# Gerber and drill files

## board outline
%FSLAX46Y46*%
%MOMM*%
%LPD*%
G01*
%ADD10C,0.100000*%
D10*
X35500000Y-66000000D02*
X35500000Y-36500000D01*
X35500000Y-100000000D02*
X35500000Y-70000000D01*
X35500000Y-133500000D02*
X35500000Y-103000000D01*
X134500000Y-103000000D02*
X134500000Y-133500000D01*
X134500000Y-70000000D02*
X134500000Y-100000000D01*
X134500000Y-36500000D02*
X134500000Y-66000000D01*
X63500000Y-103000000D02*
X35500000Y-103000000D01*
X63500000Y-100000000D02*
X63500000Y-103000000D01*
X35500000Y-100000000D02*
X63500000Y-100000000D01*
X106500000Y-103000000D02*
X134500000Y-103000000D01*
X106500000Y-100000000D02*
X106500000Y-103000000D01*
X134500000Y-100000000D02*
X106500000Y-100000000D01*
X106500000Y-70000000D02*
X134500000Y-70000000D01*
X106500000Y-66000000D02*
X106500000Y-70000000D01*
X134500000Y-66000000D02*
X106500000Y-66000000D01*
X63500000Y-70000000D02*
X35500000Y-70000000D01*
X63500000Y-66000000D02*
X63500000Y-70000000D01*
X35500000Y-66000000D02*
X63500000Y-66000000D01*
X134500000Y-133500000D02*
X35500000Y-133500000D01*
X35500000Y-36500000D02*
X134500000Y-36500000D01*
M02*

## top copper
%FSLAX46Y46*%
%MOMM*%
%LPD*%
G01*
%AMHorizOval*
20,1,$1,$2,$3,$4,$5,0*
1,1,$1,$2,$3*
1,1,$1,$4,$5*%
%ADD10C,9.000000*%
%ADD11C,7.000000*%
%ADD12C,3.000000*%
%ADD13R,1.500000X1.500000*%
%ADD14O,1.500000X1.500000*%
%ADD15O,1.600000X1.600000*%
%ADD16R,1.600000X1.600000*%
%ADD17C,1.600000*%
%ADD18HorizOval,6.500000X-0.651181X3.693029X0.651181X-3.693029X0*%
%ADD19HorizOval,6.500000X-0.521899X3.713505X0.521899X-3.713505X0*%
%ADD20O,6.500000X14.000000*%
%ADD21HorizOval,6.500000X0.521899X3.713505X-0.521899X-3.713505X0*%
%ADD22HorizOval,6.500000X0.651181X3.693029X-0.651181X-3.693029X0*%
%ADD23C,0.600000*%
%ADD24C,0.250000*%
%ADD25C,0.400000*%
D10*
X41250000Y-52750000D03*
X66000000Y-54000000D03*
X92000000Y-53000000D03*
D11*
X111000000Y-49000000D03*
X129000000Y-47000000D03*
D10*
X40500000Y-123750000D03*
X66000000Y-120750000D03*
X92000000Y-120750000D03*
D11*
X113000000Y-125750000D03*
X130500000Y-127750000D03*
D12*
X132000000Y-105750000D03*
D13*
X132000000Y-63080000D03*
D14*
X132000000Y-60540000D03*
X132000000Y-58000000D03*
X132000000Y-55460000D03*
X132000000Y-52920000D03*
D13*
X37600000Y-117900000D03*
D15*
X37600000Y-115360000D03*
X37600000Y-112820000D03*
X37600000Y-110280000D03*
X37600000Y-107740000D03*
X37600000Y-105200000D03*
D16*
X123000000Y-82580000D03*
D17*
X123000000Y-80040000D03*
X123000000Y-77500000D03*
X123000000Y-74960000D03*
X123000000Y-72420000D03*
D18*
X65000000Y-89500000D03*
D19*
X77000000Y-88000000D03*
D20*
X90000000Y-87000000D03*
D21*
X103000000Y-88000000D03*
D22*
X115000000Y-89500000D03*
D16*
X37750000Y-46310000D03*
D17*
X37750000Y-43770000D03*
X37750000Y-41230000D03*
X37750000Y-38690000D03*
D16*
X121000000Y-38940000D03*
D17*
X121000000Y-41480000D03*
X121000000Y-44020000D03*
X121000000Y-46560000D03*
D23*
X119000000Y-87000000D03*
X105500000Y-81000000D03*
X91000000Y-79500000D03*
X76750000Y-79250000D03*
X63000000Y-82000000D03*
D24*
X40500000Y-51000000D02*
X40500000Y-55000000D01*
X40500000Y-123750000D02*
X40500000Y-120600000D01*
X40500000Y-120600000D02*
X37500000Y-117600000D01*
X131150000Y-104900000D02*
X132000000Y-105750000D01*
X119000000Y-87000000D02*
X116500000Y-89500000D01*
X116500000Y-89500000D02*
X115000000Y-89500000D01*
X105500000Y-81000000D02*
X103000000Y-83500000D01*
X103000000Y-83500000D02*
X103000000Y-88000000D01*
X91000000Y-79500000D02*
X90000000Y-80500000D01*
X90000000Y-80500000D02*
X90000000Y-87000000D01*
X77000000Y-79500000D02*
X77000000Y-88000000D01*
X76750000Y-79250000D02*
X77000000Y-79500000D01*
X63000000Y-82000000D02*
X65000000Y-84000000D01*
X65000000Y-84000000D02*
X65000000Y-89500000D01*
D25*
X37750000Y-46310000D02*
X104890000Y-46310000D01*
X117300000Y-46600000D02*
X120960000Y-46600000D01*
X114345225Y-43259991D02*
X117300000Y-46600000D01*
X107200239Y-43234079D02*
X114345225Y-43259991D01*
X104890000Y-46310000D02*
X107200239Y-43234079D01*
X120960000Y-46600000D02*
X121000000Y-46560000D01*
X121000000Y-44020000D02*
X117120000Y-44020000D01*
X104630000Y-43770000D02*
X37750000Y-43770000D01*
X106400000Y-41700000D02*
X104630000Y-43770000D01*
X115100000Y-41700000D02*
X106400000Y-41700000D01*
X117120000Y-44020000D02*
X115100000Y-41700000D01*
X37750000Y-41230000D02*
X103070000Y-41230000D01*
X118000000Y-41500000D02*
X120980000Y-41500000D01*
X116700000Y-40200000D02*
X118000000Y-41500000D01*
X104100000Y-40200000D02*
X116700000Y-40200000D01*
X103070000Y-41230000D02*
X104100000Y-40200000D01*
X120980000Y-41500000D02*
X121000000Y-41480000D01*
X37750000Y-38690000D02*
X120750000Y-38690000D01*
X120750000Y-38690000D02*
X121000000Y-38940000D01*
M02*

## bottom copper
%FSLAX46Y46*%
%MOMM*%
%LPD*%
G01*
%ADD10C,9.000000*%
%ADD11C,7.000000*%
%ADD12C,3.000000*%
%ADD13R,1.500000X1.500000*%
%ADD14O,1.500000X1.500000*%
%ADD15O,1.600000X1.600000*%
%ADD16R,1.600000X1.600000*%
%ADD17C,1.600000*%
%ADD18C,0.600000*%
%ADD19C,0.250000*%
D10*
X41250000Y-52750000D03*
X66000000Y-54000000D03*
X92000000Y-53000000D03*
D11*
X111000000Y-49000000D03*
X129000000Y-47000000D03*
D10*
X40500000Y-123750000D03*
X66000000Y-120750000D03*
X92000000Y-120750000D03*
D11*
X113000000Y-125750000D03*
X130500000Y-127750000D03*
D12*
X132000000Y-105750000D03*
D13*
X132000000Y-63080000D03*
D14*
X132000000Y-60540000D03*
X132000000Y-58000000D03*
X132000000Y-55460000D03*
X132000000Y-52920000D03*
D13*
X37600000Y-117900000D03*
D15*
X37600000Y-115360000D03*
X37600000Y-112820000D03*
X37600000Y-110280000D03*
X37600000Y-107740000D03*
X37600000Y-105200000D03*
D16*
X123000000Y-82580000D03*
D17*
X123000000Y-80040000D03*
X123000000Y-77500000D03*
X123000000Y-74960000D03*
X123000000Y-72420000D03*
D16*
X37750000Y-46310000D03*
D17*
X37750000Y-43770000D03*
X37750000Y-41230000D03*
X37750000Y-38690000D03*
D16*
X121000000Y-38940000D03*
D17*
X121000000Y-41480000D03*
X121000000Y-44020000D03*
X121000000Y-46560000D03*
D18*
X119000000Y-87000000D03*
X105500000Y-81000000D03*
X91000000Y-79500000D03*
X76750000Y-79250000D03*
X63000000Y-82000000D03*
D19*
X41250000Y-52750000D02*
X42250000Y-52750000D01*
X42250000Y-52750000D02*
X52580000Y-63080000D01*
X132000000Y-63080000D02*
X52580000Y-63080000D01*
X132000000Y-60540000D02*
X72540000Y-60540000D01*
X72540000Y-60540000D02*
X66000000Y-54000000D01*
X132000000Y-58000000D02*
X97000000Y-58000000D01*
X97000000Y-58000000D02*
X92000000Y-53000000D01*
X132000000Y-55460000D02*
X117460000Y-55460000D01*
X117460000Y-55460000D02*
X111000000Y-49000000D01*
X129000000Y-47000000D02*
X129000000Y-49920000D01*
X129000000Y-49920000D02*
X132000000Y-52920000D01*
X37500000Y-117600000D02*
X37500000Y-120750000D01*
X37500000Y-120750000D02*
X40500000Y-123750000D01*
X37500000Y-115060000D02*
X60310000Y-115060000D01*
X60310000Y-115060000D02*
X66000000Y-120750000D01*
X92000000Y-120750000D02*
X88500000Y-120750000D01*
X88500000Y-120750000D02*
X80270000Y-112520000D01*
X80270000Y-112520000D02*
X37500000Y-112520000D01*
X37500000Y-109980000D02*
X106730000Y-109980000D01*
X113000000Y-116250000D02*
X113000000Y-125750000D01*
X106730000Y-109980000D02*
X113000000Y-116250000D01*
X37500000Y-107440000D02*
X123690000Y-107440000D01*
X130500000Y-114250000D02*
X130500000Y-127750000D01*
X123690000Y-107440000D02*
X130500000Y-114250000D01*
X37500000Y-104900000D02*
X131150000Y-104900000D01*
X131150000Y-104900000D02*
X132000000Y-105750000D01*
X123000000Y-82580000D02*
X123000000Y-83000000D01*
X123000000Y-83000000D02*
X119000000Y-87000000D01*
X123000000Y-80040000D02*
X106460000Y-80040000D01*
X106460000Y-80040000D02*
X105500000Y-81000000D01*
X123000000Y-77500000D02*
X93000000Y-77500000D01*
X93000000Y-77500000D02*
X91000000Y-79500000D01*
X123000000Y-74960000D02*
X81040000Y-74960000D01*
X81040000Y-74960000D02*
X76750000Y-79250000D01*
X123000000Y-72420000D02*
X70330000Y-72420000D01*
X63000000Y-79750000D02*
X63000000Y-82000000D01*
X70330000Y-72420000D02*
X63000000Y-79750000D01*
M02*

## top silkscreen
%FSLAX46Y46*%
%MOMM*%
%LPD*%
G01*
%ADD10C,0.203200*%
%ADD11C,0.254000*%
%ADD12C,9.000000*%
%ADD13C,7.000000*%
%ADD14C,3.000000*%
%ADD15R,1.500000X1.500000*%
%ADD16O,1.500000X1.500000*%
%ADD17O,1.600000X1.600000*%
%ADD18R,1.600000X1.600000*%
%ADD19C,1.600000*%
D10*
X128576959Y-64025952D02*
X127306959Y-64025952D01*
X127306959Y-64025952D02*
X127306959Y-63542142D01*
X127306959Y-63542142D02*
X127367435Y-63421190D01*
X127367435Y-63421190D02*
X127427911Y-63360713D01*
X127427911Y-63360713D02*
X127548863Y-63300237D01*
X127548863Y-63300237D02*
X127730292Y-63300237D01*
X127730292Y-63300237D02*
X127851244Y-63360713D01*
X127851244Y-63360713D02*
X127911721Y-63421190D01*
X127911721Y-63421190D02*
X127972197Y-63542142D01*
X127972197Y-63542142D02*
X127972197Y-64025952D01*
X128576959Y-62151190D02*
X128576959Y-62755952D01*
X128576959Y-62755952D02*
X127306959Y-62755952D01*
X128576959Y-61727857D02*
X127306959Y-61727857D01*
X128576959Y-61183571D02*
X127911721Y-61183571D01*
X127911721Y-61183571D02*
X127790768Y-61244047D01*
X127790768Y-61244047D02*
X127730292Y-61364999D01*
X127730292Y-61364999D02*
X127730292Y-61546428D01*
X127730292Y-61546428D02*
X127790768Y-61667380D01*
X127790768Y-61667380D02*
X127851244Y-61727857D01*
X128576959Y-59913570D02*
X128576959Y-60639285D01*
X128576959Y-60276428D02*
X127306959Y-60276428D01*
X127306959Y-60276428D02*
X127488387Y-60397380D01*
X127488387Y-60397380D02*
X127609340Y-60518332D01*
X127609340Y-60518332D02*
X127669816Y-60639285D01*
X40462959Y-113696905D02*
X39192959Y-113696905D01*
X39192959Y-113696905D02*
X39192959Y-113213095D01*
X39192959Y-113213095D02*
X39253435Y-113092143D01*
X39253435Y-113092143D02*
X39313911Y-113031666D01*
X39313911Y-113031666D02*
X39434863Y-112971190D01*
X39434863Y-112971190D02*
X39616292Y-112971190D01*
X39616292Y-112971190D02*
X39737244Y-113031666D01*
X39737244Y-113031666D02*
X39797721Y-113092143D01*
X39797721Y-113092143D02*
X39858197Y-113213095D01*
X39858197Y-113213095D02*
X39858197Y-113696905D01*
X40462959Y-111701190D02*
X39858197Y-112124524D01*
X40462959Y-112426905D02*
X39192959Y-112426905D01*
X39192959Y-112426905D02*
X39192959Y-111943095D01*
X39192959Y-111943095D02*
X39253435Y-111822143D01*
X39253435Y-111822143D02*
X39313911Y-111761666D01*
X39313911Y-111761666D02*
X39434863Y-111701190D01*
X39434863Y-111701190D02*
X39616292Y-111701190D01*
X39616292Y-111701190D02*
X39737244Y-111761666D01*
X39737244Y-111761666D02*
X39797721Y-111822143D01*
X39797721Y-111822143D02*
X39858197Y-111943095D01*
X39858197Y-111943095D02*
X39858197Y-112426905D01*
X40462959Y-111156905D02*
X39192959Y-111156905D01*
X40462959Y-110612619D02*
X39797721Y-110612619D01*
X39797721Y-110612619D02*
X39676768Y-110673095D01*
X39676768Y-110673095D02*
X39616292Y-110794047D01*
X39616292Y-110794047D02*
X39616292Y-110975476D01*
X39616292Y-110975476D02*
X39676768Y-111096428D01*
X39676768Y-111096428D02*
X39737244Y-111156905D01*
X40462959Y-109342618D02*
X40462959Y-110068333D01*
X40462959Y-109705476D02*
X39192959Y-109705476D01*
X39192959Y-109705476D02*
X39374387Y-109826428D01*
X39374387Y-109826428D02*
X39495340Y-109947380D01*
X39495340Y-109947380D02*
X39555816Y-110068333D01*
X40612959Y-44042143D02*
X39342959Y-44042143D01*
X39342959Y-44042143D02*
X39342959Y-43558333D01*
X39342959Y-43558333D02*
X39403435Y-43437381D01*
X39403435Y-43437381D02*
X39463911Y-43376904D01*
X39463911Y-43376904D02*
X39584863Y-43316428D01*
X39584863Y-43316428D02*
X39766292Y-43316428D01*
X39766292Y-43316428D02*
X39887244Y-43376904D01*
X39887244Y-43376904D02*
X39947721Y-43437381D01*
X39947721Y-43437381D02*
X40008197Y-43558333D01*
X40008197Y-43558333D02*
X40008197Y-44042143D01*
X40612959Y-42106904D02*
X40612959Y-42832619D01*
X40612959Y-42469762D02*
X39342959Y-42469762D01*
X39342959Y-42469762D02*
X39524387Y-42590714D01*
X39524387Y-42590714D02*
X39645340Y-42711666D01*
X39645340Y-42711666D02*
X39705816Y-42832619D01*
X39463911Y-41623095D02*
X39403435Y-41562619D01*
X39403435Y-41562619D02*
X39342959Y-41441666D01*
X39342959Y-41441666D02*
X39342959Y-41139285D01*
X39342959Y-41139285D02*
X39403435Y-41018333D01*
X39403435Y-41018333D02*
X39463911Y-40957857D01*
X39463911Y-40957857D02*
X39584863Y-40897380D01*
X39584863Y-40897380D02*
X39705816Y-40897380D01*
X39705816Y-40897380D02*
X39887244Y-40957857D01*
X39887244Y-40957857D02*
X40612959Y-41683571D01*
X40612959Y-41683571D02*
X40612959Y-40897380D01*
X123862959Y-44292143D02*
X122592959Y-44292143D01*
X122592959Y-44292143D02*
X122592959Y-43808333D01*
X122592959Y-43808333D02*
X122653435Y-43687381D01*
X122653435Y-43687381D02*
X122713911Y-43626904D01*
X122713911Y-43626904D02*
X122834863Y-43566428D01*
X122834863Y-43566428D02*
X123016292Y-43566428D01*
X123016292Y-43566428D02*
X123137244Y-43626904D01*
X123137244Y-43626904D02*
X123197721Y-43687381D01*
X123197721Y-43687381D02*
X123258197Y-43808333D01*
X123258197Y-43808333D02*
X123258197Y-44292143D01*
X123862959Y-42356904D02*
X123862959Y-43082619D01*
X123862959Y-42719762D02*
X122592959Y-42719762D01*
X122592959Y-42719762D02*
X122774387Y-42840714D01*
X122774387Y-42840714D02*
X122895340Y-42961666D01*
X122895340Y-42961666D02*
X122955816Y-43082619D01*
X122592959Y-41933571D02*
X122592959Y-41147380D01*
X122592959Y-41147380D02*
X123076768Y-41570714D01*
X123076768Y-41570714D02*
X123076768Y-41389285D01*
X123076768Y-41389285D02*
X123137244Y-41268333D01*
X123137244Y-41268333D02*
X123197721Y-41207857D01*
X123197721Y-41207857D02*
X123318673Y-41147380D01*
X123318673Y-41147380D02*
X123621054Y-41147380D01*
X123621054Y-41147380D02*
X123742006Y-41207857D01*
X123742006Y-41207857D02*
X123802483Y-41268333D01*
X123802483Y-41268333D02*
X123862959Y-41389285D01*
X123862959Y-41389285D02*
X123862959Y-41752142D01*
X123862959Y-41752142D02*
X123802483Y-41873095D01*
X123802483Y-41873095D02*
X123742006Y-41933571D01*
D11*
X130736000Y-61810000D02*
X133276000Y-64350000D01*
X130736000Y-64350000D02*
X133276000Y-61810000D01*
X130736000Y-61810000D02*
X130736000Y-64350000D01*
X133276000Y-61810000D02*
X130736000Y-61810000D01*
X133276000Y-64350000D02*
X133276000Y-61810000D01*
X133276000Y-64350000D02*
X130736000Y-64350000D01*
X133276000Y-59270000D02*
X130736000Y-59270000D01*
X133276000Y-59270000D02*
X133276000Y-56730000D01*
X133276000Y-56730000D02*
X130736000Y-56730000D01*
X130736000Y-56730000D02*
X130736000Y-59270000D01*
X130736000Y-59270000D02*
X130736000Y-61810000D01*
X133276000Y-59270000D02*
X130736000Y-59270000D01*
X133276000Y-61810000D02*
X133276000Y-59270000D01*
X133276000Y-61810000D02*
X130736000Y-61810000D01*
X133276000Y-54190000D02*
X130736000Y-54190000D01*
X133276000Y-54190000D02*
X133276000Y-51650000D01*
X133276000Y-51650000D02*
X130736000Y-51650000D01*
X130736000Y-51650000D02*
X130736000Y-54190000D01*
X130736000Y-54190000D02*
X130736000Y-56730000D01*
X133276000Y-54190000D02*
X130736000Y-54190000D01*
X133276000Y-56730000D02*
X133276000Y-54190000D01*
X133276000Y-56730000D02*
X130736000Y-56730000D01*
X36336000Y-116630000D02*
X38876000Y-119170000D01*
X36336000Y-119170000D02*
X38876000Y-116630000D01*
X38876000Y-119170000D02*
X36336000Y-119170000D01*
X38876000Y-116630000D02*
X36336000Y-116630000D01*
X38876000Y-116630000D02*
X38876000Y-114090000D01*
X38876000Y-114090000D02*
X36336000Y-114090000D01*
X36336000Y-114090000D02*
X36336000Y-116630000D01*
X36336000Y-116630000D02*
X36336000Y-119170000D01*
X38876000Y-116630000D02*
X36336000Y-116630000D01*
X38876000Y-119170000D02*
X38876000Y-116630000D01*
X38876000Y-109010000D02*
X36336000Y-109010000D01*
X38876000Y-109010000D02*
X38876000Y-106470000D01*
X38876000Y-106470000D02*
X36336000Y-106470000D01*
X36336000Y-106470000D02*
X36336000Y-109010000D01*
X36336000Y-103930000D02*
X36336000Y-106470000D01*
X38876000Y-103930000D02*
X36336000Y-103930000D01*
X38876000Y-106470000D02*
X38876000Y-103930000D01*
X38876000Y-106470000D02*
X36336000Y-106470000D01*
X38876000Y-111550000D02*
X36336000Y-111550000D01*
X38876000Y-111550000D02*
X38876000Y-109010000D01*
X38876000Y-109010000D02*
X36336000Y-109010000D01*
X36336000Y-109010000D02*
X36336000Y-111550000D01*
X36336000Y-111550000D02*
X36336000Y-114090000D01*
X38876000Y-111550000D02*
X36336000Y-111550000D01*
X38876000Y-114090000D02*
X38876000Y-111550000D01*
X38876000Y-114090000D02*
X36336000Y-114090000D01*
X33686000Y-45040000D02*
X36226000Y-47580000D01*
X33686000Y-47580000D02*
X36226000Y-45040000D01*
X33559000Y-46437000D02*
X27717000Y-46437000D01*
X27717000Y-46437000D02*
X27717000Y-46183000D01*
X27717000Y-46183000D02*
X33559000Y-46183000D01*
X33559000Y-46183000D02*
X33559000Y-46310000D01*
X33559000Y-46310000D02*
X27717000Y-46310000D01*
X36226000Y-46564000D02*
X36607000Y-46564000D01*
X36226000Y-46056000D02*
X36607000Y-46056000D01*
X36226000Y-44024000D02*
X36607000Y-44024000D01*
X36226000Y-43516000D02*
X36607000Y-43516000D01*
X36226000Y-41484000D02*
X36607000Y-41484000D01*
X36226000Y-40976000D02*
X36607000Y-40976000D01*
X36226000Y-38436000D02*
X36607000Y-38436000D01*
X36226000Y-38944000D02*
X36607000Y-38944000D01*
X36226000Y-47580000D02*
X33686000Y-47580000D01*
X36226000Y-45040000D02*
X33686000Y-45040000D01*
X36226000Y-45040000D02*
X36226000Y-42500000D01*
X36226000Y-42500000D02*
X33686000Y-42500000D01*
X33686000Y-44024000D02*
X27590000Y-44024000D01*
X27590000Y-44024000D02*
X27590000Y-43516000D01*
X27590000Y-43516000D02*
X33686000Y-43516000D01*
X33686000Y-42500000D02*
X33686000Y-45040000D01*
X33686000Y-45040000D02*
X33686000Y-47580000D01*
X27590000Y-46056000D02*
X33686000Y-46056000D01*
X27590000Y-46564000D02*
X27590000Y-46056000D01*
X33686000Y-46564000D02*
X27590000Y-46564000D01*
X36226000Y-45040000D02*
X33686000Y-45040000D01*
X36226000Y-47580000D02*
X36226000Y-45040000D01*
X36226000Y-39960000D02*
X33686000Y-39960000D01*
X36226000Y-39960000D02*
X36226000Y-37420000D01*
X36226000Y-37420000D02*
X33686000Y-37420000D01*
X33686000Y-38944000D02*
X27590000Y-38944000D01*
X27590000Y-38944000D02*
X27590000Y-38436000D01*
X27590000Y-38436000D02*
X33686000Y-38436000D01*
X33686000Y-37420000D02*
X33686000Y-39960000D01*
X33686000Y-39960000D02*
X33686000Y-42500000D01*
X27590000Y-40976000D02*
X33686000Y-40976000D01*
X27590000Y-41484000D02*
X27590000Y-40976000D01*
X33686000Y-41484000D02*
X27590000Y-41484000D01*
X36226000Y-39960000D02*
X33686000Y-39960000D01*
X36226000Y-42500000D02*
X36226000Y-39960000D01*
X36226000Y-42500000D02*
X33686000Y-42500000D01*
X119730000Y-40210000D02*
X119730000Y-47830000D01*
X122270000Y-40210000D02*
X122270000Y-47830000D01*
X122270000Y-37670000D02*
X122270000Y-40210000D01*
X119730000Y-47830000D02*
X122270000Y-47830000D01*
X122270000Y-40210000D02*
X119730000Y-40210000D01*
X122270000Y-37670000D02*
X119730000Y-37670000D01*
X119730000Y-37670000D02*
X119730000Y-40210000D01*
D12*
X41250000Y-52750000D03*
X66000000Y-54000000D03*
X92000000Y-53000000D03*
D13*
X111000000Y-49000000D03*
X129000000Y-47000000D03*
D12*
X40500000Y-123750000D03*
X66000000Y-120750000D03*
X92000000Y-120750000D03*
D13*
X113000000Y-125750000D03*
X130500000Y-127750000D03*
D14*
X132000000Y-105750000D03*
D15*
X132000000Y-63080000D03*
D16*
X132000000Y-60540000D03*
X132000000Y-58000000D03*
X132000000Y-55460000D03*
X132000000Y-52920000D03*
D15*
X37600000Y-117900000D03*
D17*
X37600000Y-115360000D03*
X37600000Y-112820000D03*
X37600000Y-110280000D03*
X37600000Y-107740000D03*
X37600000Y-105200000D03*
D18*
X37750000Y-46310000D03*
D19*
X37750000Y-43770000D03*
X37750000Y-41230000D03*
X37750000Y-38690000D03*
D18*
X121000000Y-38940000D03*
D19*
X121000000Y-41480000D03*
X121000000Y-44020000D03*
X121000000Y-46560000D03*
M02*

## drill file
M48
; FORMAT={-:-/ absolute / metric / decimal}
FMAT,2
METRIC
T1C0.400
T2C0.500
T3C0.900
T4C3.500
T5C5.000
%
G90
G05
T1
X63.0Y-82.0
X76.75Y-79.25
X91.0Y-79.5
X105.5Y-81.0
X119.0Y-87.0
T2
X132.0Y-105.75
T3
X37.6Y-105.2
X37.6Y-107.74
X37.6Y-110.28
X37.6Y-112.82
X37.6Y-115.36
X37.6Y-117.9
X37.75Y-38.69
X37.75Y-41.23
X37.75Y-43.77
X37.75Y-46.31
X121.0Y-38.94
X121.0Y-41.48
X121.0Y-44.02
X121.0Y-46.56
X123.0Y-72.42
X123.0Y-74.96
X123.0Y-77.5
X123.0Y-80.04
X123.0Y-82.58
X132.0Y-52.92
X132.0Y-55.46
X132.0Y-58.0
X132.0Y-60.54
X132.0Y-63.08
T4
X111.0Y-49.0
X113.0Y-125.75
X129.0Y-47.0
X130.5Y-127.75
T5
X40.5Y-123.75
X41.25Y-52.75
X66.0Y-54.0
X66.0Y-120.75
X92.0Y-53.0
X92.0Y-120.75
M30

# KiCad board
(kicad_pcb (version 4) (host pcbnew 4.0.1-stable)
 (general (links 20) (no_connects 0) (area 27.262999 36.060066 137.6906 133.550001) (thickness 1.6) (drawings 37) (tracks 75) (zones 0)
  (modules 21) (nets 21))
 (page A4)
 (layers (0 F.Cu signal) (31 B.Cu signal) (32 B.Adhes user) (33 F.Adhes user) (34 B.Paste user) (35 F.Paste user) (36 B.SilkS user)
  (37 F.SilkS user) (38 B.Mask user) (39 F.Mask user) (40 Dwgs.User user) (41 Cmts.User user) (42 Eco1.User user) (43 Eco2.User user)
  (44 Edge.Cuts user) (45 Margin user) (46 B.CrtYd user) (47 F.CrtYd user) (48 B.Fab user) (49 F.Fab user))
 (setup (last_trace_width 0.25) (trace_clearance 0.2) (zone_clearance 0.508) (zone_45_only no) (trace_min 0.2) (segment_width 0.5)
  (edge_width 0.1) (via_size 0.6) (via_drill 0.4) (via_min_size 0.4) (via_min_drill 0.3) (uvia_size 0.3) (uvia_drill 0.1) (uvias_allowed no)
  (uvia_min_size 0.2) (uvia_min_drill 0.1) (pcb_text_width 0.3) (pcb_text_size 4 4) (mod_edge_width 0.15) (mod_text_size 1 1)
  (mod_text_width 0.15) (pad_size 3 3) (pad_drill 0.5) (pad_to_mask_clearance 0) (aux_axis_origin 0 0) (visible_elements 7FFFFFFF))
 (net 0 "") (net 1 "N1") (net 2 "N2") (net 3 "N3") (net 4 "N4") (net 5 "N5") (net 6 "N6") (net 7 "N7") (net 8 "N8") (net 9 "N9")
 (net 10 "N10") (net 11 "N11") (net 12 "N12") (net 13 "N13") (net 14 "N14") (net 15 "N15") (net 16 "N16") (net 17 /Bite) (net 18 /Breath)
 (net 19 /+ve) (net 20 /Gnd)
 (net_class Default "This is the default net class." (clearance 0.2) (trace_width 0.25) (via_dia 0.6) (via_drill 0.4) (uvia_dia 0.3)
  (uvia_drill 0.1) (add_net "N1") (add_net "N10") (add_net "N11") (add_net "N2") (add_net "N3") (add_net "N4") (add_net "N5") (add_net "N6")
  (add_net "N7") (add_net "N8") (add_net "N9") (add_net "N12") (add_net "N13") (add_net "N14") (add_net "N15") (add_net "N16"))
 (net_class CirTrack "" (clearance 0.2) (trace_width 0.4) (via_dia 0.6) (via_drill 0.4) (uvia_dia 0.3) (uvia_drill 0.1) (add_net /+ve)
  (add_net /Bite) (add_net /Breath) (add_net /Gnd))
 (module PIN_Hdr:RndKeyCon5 (layer F.Cu) (at 41.25 52.75)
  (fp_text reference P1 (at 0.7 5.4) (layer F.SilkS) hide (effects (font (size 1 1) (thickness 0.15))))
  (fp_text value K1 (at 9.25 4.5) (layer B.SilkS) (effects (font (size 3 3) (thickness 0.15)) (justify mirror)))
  (pad 1 thru_hole circle (at 0 0) (size 9 9) (drill 5) (layers *.Cu *.Mask F.SilkS) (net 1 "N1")))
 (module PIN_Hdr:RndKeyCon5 (layer F.Cu) (at 66 54)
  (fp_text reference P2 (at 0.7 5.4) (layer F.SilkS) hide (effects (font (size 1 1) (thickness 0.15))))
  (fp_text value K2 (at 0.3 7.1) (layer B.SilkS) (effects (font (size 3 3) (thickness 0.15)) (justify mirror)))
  (pad 1 thru_hole circle (at 0 0) (size 9 9) (drill 5) (layers *.Cu *.Mask F.SilkS) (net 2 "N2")))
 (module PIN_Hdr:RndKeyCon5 (layer F.Cu) (at 92 53)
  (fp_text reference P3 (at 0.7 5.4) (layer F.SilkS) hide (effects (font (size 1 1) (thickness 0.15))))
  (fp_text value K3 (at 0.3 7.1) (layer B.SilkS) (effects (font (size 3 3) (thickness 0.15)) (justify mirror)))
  (pad 1 thru_hole circle (at 0 0) (size 9 9) (drill 5) (layers *.Cu *.Mask F.SilkS) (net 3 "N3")))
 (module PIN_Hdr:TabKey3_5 (layer F.Cu) (at 111 49)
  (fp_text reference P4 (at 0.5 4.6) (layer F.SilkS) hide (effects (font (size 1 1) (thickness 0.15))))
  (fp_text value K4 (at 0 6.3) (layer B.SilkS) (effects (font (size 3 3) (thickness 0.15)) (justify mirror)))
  (pad 1 thru_hole circle (at 0 0) (size 7 7) (drill 3.5) (layers *.Cu *.Mask F.SilkS) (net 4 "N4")))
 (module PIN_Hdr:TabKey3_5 (layer F.Cu) (at 129 47)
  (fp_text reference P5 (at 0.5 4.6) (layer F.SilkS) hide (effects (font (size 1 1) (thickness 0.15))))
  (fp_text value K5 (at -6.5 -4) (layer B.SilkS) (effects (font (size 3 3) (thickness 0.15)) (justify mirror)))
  (pad 1 thru_hole circle (at 0 0) (size 7 7) (drill 3.5) (layers *.Cu *.Mask F.SilkS) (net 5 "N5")))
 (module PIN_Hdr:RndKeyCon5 (layer F.Cu) (at 40.5 123.75)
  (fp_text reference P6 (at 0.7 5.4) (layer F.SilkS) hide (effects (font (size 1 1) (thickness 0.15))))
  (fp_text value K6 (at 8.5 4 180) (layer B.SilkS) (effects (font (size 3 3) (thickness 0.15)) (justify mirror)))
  (pad 1 thru_hole circle (at 0 0) (size 9 9) (drill 5) (layers *.Cu *.Mask F.SilkS) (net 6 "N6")))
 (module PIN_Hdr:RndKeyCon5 (layer F.Cu) (at 66 120.75)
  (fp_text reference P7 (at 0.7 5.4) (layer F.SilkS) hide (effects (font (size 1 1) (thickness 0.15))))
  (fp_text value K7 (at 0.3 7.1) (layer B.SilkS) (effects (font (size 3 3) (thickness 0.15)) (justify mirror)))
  (pad 1 thru_hole circle (at 0 0) (size 9 9) (drill 5) (layers *.Cu *.Mask F.SilkS) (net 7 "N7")))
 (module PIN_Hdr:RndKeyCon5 (layer F.Cu) (at 92 120.75)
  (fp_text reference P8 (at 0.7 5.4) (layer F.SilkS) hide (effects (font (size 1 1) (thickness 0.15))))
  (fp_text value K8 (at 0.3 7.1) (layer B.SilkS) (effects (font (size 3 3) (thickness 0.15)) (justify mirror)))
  (pad 1 thru_hole circle (at 0 0) (size 9 9) (drill 5) (layers *.Cu *.Mask F.SilkS) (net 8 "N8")))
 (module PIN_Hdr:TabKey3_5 (layer F.Cu) (at 113 125.75)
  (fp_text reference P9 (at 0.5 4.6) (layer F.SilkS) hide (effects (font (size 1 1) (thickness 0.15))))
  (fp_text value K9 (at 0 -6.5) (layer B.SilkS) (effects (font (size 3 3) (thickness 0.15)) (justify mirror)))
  (pad 1 thru_hole circle (at 0 0) (size 7 7) (drill 3.5) (layers *.Cu *.Mask F.SilkS) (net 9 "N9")))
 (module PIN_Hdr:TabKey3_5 (layer F.Cu) (at 130.5 127.75)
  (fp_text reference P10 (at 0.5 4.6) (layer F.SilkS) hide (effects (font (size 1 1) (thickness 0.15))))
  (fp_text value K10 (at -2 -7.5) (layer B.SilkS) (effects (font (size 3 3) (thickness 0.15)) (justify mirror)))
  (pad 1 thru_hole circle (at 0 0) (size 7 7) (drill 3.5) (layers *.Cu *.Mask F.SilkS) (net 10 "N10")))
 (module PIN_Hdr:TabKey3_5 (layer F.Cu) (at 132 105.75)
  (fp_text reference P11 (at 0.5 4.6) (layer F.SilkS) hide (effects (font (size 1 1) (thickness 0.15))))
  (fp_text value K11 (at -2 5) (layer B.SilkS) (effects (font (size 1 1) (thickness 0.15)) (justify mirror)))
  (pad 1 thru_hole circle (at 0 0) (size 3 3) (drill 0.5) (layers *.Cu *.Mask F.SilkS) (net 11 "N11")))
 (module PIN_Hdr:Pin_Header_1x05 (layer F.Cu) (at 132 58 90)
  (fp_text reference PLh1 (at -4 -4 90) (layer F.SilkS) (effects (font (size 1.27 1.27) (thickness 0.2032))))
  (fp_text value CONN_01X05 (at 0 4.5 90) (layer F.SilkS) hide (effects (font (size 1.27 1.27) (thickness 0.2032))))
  (fp_line (start -3.81 -1.264) (end -6.35 1.276) (layer F.SilkS) (width 0.254))
  (fp_line (start -6.35 -1.264) (end -3.81 1.276) (layer F.SilkS) (width 0.254))
  (fp_line (start -3.81 -1.264) (end -6.35 -1.264) (layer F.SilkS) (width 0.254))
  (fp_line (start -3.81 1.276) (end -3.81 -1.264) (layer F.SilkS) (width 0.254))
  (fp_line (start -6.35 1.276) (end -3.81 1.276) (layer F.SilkS) (width 0.254))
  (fp_line (start -6.35 1.276) (end -6.35 -1.264) (layer F.SilkS) (width 0.254))
  (fp_line (start -1.27 1.276) (end -1.27 -1.264) (layer F.SilkS) (width 0.254))
  (fp_line (start -1.27 1.276) (end 1.27 1.276) (layer F.SilkS) (width 0.254))
  (fp_line (start 1.27 1.276) (end 1.27 -1.264) (layer F.SilkS) (width 0.254))
  (fp_line (start 1.27 -1.264) (end -1.27 -1.264) (layer F.SilkS) (width 0.254))
  (fp_line (start -1.27 -1.264) (end -3.81 -1.264) (layer F.SilkS) (width 0.254))
  (fp_line (start -1.27 1.276) (end -1.27 -1.264) (layer F.SilkS) (width 0.254))
  (fp_line (start -3.81 1.276) (end -1.27 1.276) (layer F.SilkS) (width 0.254))
  (fp_line (start -3.81 1.276) (end -3.81 -1.264) (layer F.SilkS) (width 0.254))
  (fp_line (start 3.81 1.276) (end 3.81 -1.264) (layer F.SilkS) (width 0.254))
  (fp_line (start 3.81 1.276) (end 6.35 1.276) (layer F.SilkS) (width 0.254))
  (fp_line (start 6.35 1.276) (end 6.35 -1.264) (layer F.SilkS) (width 0.254))
  (fp_line (start 6.35 -1.264) (end 3.81 -1.264) (layer F.SilkS) (width 0.254))
  (fp_line (start 3.81 -1.264) (end 1.27 -1.264) (layer F.SilkS) (width 0.254))
  (fp_line (start 3.81 1.276) (end 3.81 -1.264) (layer F.SilkS) (width 0.254))
  (fp_line (start 1.27 1.276) (end 3.81 1.276) (layer F.SilkS) (width 0.254))
  (fp_line (start 1.27 1.276) (end 1.27 -1.264) (layer F.SilkS) (width 0.254))
  (pad 1 thru_hole rect (at -5.08 0 90) (size 1.5 1.5) (drill 0.9) (layers *.Cu *.Mask F.SilkS) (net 1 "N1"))
  (pad 2 thru_hole oval (at -2.54 0 90) (size 1.5 1.5) (drill 0.9) (layers *.Cu *.Mask F.SilkS) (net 2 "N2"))
  (pad 3 thru_hole oval (at 0 0 90) (size 1.5 1.5) (drill 0.9) (layers *.Cu *.Mask F.SilkS) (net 3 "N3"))
  (pad 4 thru_hole oval (at 2.54 0 90) (size 1.5 1.5) (drill 0.9) (layers *.Cu *.Mask F.SilkS) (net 4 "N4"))
  (pad 5 thru_hole oval (at 5.08 0 90) (size 1.5 1.5) (drill 0.9) (layers *.Cu *.Mask F.SilkS) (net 5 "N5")))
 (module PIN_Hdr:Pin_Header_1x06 (layer F.Cu) (at 37.6 111.55 90)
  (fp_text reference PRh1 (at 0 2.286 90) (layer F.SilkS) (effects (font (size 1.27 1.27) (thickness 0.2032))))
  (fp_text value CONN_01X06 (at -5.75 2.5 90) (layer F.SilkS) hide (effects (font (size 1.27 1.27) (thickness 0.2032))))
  (fp_line (start -5.08 -1.264) (end -7.62 1.276) (layer F.SilkS) (width 0.254))
  (fp_line (start -7.62 -1.264) (end -5.08 1.276) (layer F.SilkS) (width 0.254))
  (fp_line (start -7.62 1.276) (end -7.62 -1.264) (layer F.SilkS) (width 0.254))
  (fp_line (start -5.08 1.276) (end -5.08 -1.264) (layer F.SilkS) (width 0.254))
  (fp_line (start -5.08 1.276) (end -2.54 1.276) (layer F.SilkS) (width 0.254))
  (fp_line (start -2.54 1.276) (end -2.54 -1.264) (layer F.SilkS) (width 0.254))
  (fp_line (start -2.54 -1.264) (end -5.08 -1.264) (layer F.SilkS) (width 0.254))
  (fp_line (start -5.08 -1.264) (end -7.62 -1.264) (layer F.SilkS) (width 0.254))
  (fp_line (start -5.08 1.276) (end -5.08 -1.264) (layer F.SilkS) (width 0.254))
  (fp_line (start -7.62 1.276) (end -5.08 1.276) (layer F.SilkS) (width 0.254))
  (fp_line (start 2.54 1.276) (end 2.54 -1.264) (layer F.SilkS) (width 0.254))
  (fp_line (start 2.54 1.276) (end 5.08 1.276) (layer F.SilkS) (width 0.254))
  (fp_line (start 5.08 1.276) (end 5.08 -1.264) (layer F.SilkS) (width 0.254))
  (fp_line (start 5.08 -1.264) (end 2.54 -1.264) (layer F.SilkS) (width 0.254))
  (fp_line (start 7.62 -1.264) (end 5.08 -1.264) (layer F.SilkS) (width 0.254))
  (fp_line (start 7.62 1.276) (end 7.62 -1.264) (layer F.SilkS) (width 0.254))
  (fp_line (start 5.08 1.276) (end 7.62 1.276) (layer F.SilkS) (width 0.254))
  (fp_line (start 5.08 1.276) (end 5.08 -1.264) (layer F.SilkS) (width 0.254))
  (fp_line (start 0 1.276) (end 0 -1.264) (layer F.SilkS) (width 0.254))
  (fp_line (start 0 1.276) (end 2.54 1.276) (layer F.SilkS) (width 0.254))
  (fp_line (start 2.54 1.276) (end 2.54 -1.264) (layer F.SilkS) (width 0.254))
  (fp_line (start 2.54 -1.264) (end 0 -1.264) (layer F.SilkS) (width 0.254))
  (fp_line (start 0 -1.264) (end -2.54 -1.264) (layer F.SilkS) (width 0.254))
  (fp_line (start 0 1.276) (end 0 -1.264) (layer F.SilkS) (width 0.254))
  (fp_line (start -2.54 1.276) (end 0 1.276) (layer F.SilkS) (width 0.254))
  (fp_line (start -2.54 1.276) (end -2.54 -1.264) (layer F.SilkS) (width 0.254))
  (pad 1 thru_hole rect (at -6.35 0 90) (size 1.5 1.5) (drill 0.9) (layers *.Cu *.Mask F.SilkS) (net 6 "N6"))
  (pad 2 thru_hole oval (at -3.81 0 90) (size 1.6 1.6) (drill 0.9) (layers *.Cu *.Mask F.SilkS) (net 7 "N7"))
  (pad 3 thru_hole oval (at -1.27 0 90) (size 1.6 1.6) (drill 0.9) (layers *.Cu *.Mask F.SilkS) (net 8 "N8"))
  (pad 4 thru_hole oval (at 1.27 0 90) (size 1.6 1.6) (drill 0.9) (layers *.Cu *.Mask F.SilkS) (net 9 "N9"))
  (pad 5 thru_hole oval (at 3.81 0 90) (size 1.6 1.6) (drill 0.9) (layers *.Cu *.Mask F.SilkS) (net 10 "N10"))
  (pad 6 thru_hole oval (at 6.35 0 90) (size 1.6 1.6) (drill 0.9) (layers *.Cu *.Mask F.SilkS) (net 11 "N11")))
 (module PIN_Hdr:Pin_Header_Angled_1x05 (layer B.Cu) (at 123 77.5 90)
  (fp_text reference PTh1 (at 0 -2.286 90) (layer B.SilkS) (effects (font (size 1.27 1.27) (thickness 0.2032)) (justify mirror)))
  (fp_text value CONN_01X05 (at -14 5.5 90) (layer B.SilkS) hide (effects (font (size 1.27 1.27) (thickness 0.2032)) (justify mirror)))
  (pad 1 thru_hole rect (at -5.08 0 90) (size 1.6 1.6) (drill 0.9) (layers *.Cu *.Mask B.SilkS) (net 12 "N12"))
  (pad 2 thru_hole circle (at -2.54 0 90) (size 1.6 1.6) (drill 0.9) (layers *.Cu *.Mask B.SilkS) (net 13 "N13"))
  (pad 3 thru_hole circle (at 0 0 90) (size 1.6 1.6) (drill 0.9) (layers *.Cu *.Mask B.SilkS) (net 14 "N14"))
  (pad 4 thru_hole circle (at 2.54 0 90) (size 1.6 1.6) (drill 0.9) (layers *.Cu *.Mask B.SilkS) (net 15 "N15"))
  (pad 5 thru_hole circle (at 5.08 0 90) (size 1.6 1.6) (drill 0.9) (layers *.Cu *.Mask B.SilkS) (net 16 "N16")))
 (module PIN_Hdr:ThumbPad (layer F.Cu) (at 65 89.5 100)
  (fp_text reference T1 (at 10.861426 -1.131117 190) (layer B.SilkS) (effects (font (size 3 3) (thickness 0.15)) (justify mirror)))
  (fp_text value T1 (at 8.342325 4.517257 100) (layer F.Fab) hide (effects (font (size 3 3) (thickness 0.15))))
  (pad 1 smd oval (at 0 0 100) (size 14 6.5) (layers F.Cu F.Paste F.Mask) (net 16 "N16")))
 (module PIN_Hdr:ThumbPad (layer F.Cu) (at 77 88 98)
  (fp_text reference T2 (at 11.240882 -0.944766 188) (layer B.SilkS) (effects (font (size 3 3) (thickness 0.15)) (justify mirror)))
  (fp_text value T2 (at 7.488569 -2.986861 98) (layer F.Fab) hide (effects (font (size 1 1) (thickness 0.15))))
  (pad 1 smd oval (at 0 0 98) (size 14 6.5) (layers F.Cu F.Paste F.Mask) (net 15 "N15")))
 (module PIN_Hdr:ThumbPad (layer F.Cu) (at 90 87 90)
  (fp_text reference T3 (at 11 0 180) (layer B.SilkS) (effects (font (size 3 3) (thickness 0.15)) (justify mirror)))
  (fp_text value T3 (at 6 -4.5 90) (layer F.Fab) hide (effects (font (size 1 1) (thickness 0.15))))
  (pad 1 smd oval (at 0 0 90) (size 14 6.5) (layers F.Cu F.Paste F.Mask) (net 14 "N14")))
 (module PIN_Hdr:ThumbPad (layer F.Cu) (at 103 88 82)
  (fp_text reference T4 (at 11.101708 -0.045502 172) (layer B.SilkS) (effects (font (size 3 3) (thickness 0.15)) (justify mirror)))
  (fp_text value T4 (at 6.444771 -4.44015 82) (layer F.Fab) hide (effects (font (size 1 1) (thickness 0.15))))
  (pad 1 smd oval (at 0 0 82) (size 14 6.5) (layers F.Cu F.Paste F.Mask) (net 13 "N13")))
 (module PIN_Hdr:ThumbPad (layer F.Cu) (at 115 89.5 80)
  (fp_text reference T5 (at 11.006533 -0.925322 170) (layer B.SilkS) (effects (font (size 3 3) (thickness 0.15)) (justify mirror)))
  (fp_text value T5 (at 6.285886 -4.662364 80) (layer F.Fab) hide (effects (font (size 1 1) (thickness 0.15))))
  (pad 1 smd oval (at 0 0 80) (size 14 6.5) (layers F.Cu F.Paste F.Mask) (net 12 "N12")))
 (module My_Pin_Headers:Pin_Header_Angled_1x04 (layer F.Cu) (at 37.75 42.5 90)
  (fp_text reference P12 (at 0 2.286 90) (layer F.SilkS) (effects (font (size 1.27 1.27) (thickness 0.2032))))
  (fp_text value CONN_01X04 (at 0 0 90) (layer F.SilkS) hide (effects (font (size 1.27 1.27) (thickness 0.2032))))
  (fp_line (start -2.54 -4.064) (end -5.08 -1.524) (layer F.SilkS) (width 0.254))
  (fp_line (start -5.08 -4.064) (end -2.54 -1.524) (layer F.SilkS) (width 0.254))
  (fp_line (start -3.937 -4.191) (end -3.937 -10.033) (layer F.SilkS) (width 0.254))
  (fp_line (start -3.937 -10.033) (end -3.683 -10.033) (layer F.SilkS) (width 0.254))
  (fp_line (start -3.683 -10.033) (end -3.683 -4.191) (layer F.SilkS) (width 0.254))
  (fp_line (start -3.683 -4.191) (end -3.81 -4.191) (layer F.SilkS) (width 0.254))
  (fp_line (start -3.81 -4.191) (end -3.81 -10.033) (layer F.SilkS) (width 0.254))
  (fp_line (start -4.064 -1.524) (end -4.064 -1.143) (layer F.SilkS) (width 0.254))
  (fp_line (start -3.556 -1.524) (end -3.556 -1.143) (layer F.SilkS) (width 0.254))
  (fp_line (start -1.524 -1.524) (end -1.524 -1.143) (layer F.SilkS) (width 0.254))
  (fp_line (start -1.016 -1.524) (end -1.016 -1.143) (layer F.SilkS) (width 0.254))
  (fp_line (start 1.016 -1.524) (end 1.016 -1.143) (layer F.SilkS) (width 0.254))
  (fp_line (start 1.524 -1.524) (end 1.524 -1.143) (layer F.SilkS) (width 0.254))
  (fp_line (start 4.064 -1.524) (end 4.064 -1.143) (layer F.SilkS) (width 0.254))
  (fp_line (start 3.556 -1.524) (end 3.556 -1.143) (layer F.SilkS) (width 0.254))
  (fp_line (start -5.08 -1.524) (end -5.08 -4.064) (layer F.SilkS) (width 0.254))
  (fp_line (start -2.54 -1.524) (end -2.54 -4.064) (layer F.SilkS) (width 0.254))
  (fp_line (start -2.54 -1.524) (end 0 -1.524) (layer F.SilkS) (width 0.254))
  (fp_line (start 0 -1.524) (end 0 -4.064) (layer F.SilkS) (width 0.254))
  (fp_line (start -1.524 -4.064) (end -1.524 -10.16) (layer F.SilkS) (width 0.254))
  (fp_line (start -1.524 -10.16) (end -1.016 -10.16) (layer F.SilkS) (width 0.254))
  (fp_line (start -1.016 -10.16) (end -1.016 -4.064) (layer F.SilkS) (width 0.254))
  (fp_line (start 0 -4.064) (end -2.54 -4.064) (layer F.SilkS) (width 0.254))
  (fp_line (start -2.54 -4.064) (end -5.08 -4.064) (layer F.SilkS) (width 0.254))
  (fp_line (start -3.556 -10.16) (end -3.556 -4.064) (layer F.SilkS) (width 0.254))
  (fp_line (start -4.064 -10.16) (end -3.556 -10.16) (layer F.SilkS) (width 0.254))
  (fp_line (start -4.064 -4.064) (end -4.064 -10.16) (layer F.SilkS) (width 0.254))
  (fp_line (start -2.54 -1.524) (end -2.54 -4.064) (layer F.SilkS) (width 0.254))
  (fp_line (start -5.08 -1.524) (end -2.54 -1.524) (layer F.SilkS) (width 0.254))
  (fp_line (start 2.54 -1.524) (end 2.54 -4.064) (layer F.SilkS) (width 0.254))
  (fp_line (start 2.54 -1.524) (end 5.08 -1.524) (layer F.SilkS) (width 0.254))
  (fp_line (start 5.08 -1.524) (end 5.08 -4.064) (layer F.SilkS) (width 0.254))
  (fp_line (start 3.556 -4.064) (end 3.556 -10.16) (layer F.SilkS) (width 0.254))
  (fp_line (start 3.556 -10.16) (end 4.064 -10.16) (layer F.SilkS) (width 0.254))
  (fp_line (start 4.064 -10.16) (end 4.064 -4.064) (layer F.SilkS) (width 0.254))
  (fp_line (start 5.08 -4.064) (end 2.54 -4.064) (layer F.SilkS) (width 0.254))
  (fp_line (start 2.54 -4.064) (end 0 -4.064) (layer F.SilkS) (width 0.254))
  (fp_line (start 1.524 -10.16) (end 1.524 -4.064) (layer F.SilkS) (width 0.254))
  (fp_line (start 1.016 -10.16) (end 1.524 -10.16) (layer F.SilkS) (width 0.254))
  (fp_line (start 1.016 -4.064) (end 1.016 -10.16) (layer F.SilkS) (width 0.254))
  (fp_line (start 2.54 -1.524) (end 2.54 -4.064) (layer F.SilkS) (width 0.254))
  (fp_line (start 0 -1.524) (end 2.54 -1.524) (layer F.SilkS) (width 0.254))
  (fp_line (start 0 -1.524) (end 0 -4.064) (layer F.SilkS) (width 0.254))
  (pad 1 thru_hole rect (at -3.81 0 90) (size 1.6 1.6) (drill 0.9) (layers *.Cu *.Mask F.SilkS) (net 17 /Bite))
  (pad 2 thru_hole circle (at -1.27 0 90) (size 1.6 1.6) (drill 0.9) (layers *.Cu *.Mask F.SilkS) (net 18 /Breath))
  (pad 3 thru_hole circle (at 1.27 0 90) (size 1.6 1.6) (drill 0.9) (layers *.Cu *.Mask F.SilkS) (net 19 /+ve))
  (pad 4 thru_hole circle (at 3.81 0 90) (size 1.6 1.6) (drill 0.9) (layers *.Cu *.Mask F.SilkS) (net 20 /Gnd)))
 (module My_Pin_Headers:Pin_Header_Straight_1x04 (layer F.Cu) (at 121 42.75 270)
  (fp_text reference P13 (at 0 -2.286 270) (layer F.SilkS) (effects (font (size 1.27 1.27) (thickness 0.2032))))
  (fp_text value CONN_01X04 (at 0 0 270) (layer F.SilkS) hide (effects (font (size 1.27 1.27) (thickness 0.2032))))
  (fp_line (start -2.54 1.27) (end 5.08 1.27) (layer F.SilkS) (width 0.254))
  (fp_line (start -2.54 -1.27) (end 5.08 -1.27) (layer F.SilkS) (width 0.254))
  (fp_line (start -5.08 -1.27) (end -2.54 -1.27) (layer F.SilkS) (width 0.254))
  (fp_line (start 5.08 1.27) (end 5.08 -1.27) (layer F.SilkS) (width 0.254))
  (fp_line (start -2.54 -1.27) (end -2.54 1.27) (layer F.SilkS) (width 0.254))
  (fp_line (start -5.08 -1.27) (end -5.08 1.27) (layer F.SilkS) (width 0.254))
  (fp_line (start -5.08 1.27) (end -2.54 1.27) (layer F.SilkS) (width 0.254))
  (pad 1 thru_hole rect (at -3.81 0 270) (size 1.6 1.6) (drill 0.9) (layers *.Cu *.Mask F.SilkS) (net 20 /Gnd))
  (pad 2 thru_hole circle (at -1.27 0 270) (size 1.6 1.6) (drill 0.9) (layers *.Cu *.Mask F.SilkS) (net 19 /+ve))
  (pad 3 thru_hole circle (at 1.27 0 270) (size 1.6 1.6) (drill 0.9) (layers *.Cu *.Mask F.SilkS) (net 18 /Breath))
  (pad 4 thru_hole circle (at 3.81 0 270) (size 1.6 1.6) (drill 0.9) (layers *.Cu *.Mask F.SilkS) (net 17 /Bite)))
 (gr_line (start 35.5 66) (end 35.5 36.5) (angle 90) (layer Edge.Cuts) (width 0.1))
 (gr_line (start 35.5 100) (end 35.5 70) (angle 90) (layer Edge.Cuts) (width 0.1))
 (gr_line (start 35.5 133.5) (end 35.5 103) (angle 90) (layer Edge.Cuts) (width 0.1))
 (gr_line (start 134.5 103) (end 134.5 133.5) (angle 90) (layer Edge.Cuts) (width 0.1))
 (gr_line (start 134.5 70) (end 134.5 100) (angle 90) (layer Edge.Cuts) (width 0.1))
 (gr_line (start 134.5 36.5) (end 134.5 66) (angle 90) (layer Edge.Cuts) (width 0.1))
 (gr_line (start 63.5 103) (end 35.5 103) (angle 90) (layer Edge.Cuts) (width 0.1))
 (gr_line (start 63.5 100) (end 63.5 103) (angle 90) (layer Edge.Cuts) (width 0.1))
 (gr_line (start 35.5 100) (end 63.5 100) (angle 90) (layer Edge.Cuts) (width 0.1))
 (gr_line (start 106.5 103) (end 134.5 103) (angle 90) (layer Edge.Cuts) (width 0.1))
 (gr_line (start 106.5 100) (end 106.5 103) (angle 90) (layer Edge.Cuts) (width 0.1))
 (gr_line (start 134.5 100) (end 106.5 100) (angle 90) (layer Edge.Cuts) (width 0.1))
 (gr_line (start 106.5 70) (end 134.5 70) (angle 90) (layer Edge.Cuts) (width 0.1))
 (gr_line (start 106.5 66) (end 106.5 70) (angle 90) (layer Edge.Cuts) (width 0.1))
 (gr_line (start 134.5 66) (end 106.5 66) (angle 90) (layer Edge.Cuts) (width 0.1))
 (gr_line (start 63.5 70) (end 35.5 70) (angle 90) (layer Edge.Cuts) (width 0.1))
 (gr_line (start 63.5 66) (end 63.5 70) (angle 90) (layer Edge.Cuts) (width 0.1))
 (gr_line (start 35.5 66) (end 63.5 66) (angle 90) (layer Edge.Cuts) (width 0.1))
 (gr_line (start 134.5 133.5) (end 35.5 133.5) (angle 90) (layer Edge.Cuts) (width 0.1))
 (gr_line (start 35.5 36.5) (end 134.5 36.5) (angle 90) (layer Edge.Cuts) (width 0.1))
 (segment (start 41.25 52.75) (end 42.25 52.75) (width 0.25) (layer B.Cu) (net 1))
 (segment (start 42.25 52.75) (end 52.58 63.08) (width 0.25) (layer B.Cu) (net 1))
 (segment (start 132 63.08) (end 52.58 63.08) (width 0.25) (layer B.Cu) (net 1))
 (segment (start 40.5 51) (end 40.5 55) (width 0.25) (layer F.Cu) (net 1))
 (segment (start 132 60.54) (end 72.54 60.54) (width 0.25) (layer B.Cu) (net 2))
 (segment (start 72.54 60.54) (end 66 54) (width 0.25) (layer B.Cu) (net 2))
 (segment (start 132 58) (end 97 58) (width 0.25) (layer B.Cu) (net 3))
 (segment (start 97 58) (end 92 53) (width 0.25) (layer B.Cu) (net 3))
 (segment (start 132 55.46) (end 117.46 55.46) (width 0.25) (layer B.Cu) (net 4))
 (segment (start 117.46 55.46) (end 111 49) (width 0.25) (layer B.Cu) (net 4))
 (segment (start 129 47) (end 129 49.92) (width 0.25) (layer B.Cu) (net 5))
 (segment (start 129 49.92) (end 132 52.92) (width 0.25) (layer B.Cu) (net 5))
 (segment (start 37.5 117.6) (end 37.5 120.75) (width 0.25) (layer B.Cu) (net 6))
 (segment (start 37.5 120.75) (end 40.5 123.75) (width 0.25) (layer B.Cu) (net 6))
 (segment (start 40.5 123.75) (end 40.5 120.6) (width 0.25) (layer F.Cu) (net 6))
 (segment (start 40.5 120.6) (end 37.5 117.6) (width 0.25) (layer F.Cu) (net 6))
 (segment (start 37.5 115.06) (end 60.31 115.06) (width 0.25) (layer B.Cu) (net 7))
 (segment (start 60.31 115.06) (end 66 120.75) (width 0.25) (layer B.Cu) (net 7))
 (segment (start 92 120.75) (end 88.5 120.75) (width 0.25) (layer B.Cu) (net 8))
 (segment (start 88.5 120.75) (end 80.27 112.52) (width 0.25) (layer B.Cu) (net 8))
 (segment (start 80.27 112.52) (end 37.5 112.52) (width 0.25) (layer B.Cu) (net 8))
 (segment (start 37.5 109.98) (end 106.73 109.98) (width 0.25) (layer B.Cu) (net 9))
 (segment (start 113 116.25) (end 113 125.75) (width 0.25) (layer B.Cu) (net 9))
 (segment (start 106.73 109.98) (end 113 116.25) (width 0.25) (layer B.Cu) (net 9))
 (segment (start 37.5 107.44) (end 123.69 107.44) (width 0.25) (layer B.Cu) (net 10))
 (segment (start 130.5 114.25) (end 130.5 127.75) (width 0.25) (layer B.Cu) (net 10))
 (segment (start 123.69 107.44) (end 130.5 114.25) (width 0.25) (layer B.Cu) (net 10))
 (segment (start 37.5 104.9) (end 131.15 104.9) (width 0.25) (layer B.Cu) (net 11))
 (segment (start 131.15 104.9) (end 132 105.75) (width 0.25) (layer B.Cu) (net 11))
 (segment (start 131.15 104.9) (end 132 105.75) (width 0.25) (layer F.Cu) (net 11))
 (segment (start 123 82.58) (end 123 83) (width 0.25) (layer B.Cu) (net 12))
 (segment (start 123 83) (end 119 87) (width 0.25) (layer B.Cu) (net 12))
 (via (at 119 87) (size 0.6) (drill 0.4) (layers F.Cu B.Cu) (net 12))
 (segment (start 119 87) (end 116.5 89.5) (width 0.25) (layer F.Cu) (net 12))
 (segment (start 116.5 89.5) (end 115 89.5) (width 0.25) (layer F.Cu) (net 12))
 (segment (start 123 80.04) (end 106.46 80.04) (width 0.25) (layer B.Cu) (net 13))
 (segment (start 105.5 81) (end 103 83.5) (width 0.25) (layer F.Cu) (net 13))
 (via (at 105.5 81) (size 0.6) (drill 0.4) (layers F.Cu B.Cu) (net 13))
 (segment (start 106.46 80.04) (end 105.5 81) (width 0.25) (layer B.Cu) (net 13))
 (segment (start 103 83.5) (end 103 88) (width 0.25) (layer F.Cu) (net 13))
 (segment (start 123 77.5) (end 93 77.5) (width 0.25) (layer B.Cu) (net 14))
 (segment (start 91 79.5) (end 90 80.5) (width 0.25) (layer F.Cu) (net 14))
 (via (at 91 79.5) (size 0.6) (drill 0.4) (layers F.Cu B.Cu) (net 14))
 (segment (start 93 77.5) (end 91 79.5) (width 0.25) (layer B.Cu) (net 14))
 (segment (start 90 80.5) (end 90 87) (width 0.25) (layer F.Cu) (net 14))
 (segment (start 123 74.96) (end 81.04 74.96) (width 0.25) (layer B.Cu) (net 15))
 (segment (start 77 79.5) (end 77 88) (width 0.25) (layer F.Cu) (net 15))
 (segment (start 76.75 79.25) (end 77 79.5) (width 0.25) (layer F.Cu) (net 15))
 (via (at 76.75 79.25) (size 0.6) (drill 0.4) (layers F.Cu B.Cu) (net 15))
 (segment (start 81.04 74.96) (end 76.75 79.25) (width 0.25) (layer B.Cu) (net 15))
 (segment (start 123 72.42) (end 70.33 72.42) (width 0.25) (layer B.Cu) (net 16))
 (segment (start 63 82) (end 65 84) (width 0.25) (layer F.Cu) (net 16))
 (via (at 63 82) (size 0.6) (drill 0.4) (layers F.Cu B.Cu) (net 16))
 (segment (start 63 79.75) (end 63 82) (width 0.25) (layer B.Cu) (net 16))
 (segment (start 70.33 72.42) (end 63 79.75) (width 0.25) (layer B.Cu) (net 16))
 (segment (start 65 84) (end 65 89.5) (width 0.25) (layer F.Cu) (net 16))
 (segment (start 37.75 46.31) (end 104.89 46.31) (width 0.4) (layer F.Cu) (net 17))
 (segment (start 117.3 46.6) (end 120.96 46.6) (width 0.4) (layer F.Cu) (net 17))
 (segment (start 114.345225 43.259991) (end 117.3 46.6) (width 0.4) (layer F.Cu) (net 17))
 (segment (start 107.200239 43.234079) (end 114.345225 43.259991) (width 0.4) (layer F.Cu) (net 17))
 (segment (start 104.89 46.31) (end 107.200239 43.234079) (width 0.4) (layer F.Cu) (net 17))
 (segment (start 120.96 46.6) (end 121 46.56) (width 0.4) (layer F.Cu) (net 17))
 (segment (start 121 44.02) (end 117.12 44.02) (width 0.4) (layer F.Cu) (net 18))
 (segment (start 104.63 43.77) (end 37.75 43.77) (width 0.4) (layer F.Cu) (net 18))
 (segment (start 106.4 41.7) (end 104.63 43.77) (width 0.4) (layer F.Cu) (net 18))
 (segment (start 115.1 41.7) (end 106.4 41.7) (width 0.4) (layer F.Cu) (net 18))
 (segment (start 117.12 44.02) (end 115.1 41.7) (width 0.4) (layer F.Cu) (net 18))
 (segment (start 37.75 41.23) (end 103.07 41.23) (width 0.4) (layer F.Cu) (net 19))
 (segment (start 118 41.5) (end 120.98 41.5) (width 0.4) (layer F.Cu) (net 19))
 (segment (start 116.7 40.2) (end 118 41.5) (width 0.4) (layer F.Cu) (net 19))
 (segment (start 104.1 40.2) (end 116.7 40.2) (width 0.4) (layer F.Cu) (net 19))
 (segment (start 103.07 41.23) (end 104.1 40.2) (width 0.4) (layer F.Cu) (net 19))
 (segment (start 120.98 41.5) (end 121 41.48) (width 0.4) (layer F.Cu) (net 19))
 (segment (start 37.75 38.69) (end 120.75 38.69) (width 0.4) (layer F.Cu) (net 20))
 (segment (start 120.75 38.69) (end 121 38.94) (width 0.4) (layer F.Cu) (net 20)))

